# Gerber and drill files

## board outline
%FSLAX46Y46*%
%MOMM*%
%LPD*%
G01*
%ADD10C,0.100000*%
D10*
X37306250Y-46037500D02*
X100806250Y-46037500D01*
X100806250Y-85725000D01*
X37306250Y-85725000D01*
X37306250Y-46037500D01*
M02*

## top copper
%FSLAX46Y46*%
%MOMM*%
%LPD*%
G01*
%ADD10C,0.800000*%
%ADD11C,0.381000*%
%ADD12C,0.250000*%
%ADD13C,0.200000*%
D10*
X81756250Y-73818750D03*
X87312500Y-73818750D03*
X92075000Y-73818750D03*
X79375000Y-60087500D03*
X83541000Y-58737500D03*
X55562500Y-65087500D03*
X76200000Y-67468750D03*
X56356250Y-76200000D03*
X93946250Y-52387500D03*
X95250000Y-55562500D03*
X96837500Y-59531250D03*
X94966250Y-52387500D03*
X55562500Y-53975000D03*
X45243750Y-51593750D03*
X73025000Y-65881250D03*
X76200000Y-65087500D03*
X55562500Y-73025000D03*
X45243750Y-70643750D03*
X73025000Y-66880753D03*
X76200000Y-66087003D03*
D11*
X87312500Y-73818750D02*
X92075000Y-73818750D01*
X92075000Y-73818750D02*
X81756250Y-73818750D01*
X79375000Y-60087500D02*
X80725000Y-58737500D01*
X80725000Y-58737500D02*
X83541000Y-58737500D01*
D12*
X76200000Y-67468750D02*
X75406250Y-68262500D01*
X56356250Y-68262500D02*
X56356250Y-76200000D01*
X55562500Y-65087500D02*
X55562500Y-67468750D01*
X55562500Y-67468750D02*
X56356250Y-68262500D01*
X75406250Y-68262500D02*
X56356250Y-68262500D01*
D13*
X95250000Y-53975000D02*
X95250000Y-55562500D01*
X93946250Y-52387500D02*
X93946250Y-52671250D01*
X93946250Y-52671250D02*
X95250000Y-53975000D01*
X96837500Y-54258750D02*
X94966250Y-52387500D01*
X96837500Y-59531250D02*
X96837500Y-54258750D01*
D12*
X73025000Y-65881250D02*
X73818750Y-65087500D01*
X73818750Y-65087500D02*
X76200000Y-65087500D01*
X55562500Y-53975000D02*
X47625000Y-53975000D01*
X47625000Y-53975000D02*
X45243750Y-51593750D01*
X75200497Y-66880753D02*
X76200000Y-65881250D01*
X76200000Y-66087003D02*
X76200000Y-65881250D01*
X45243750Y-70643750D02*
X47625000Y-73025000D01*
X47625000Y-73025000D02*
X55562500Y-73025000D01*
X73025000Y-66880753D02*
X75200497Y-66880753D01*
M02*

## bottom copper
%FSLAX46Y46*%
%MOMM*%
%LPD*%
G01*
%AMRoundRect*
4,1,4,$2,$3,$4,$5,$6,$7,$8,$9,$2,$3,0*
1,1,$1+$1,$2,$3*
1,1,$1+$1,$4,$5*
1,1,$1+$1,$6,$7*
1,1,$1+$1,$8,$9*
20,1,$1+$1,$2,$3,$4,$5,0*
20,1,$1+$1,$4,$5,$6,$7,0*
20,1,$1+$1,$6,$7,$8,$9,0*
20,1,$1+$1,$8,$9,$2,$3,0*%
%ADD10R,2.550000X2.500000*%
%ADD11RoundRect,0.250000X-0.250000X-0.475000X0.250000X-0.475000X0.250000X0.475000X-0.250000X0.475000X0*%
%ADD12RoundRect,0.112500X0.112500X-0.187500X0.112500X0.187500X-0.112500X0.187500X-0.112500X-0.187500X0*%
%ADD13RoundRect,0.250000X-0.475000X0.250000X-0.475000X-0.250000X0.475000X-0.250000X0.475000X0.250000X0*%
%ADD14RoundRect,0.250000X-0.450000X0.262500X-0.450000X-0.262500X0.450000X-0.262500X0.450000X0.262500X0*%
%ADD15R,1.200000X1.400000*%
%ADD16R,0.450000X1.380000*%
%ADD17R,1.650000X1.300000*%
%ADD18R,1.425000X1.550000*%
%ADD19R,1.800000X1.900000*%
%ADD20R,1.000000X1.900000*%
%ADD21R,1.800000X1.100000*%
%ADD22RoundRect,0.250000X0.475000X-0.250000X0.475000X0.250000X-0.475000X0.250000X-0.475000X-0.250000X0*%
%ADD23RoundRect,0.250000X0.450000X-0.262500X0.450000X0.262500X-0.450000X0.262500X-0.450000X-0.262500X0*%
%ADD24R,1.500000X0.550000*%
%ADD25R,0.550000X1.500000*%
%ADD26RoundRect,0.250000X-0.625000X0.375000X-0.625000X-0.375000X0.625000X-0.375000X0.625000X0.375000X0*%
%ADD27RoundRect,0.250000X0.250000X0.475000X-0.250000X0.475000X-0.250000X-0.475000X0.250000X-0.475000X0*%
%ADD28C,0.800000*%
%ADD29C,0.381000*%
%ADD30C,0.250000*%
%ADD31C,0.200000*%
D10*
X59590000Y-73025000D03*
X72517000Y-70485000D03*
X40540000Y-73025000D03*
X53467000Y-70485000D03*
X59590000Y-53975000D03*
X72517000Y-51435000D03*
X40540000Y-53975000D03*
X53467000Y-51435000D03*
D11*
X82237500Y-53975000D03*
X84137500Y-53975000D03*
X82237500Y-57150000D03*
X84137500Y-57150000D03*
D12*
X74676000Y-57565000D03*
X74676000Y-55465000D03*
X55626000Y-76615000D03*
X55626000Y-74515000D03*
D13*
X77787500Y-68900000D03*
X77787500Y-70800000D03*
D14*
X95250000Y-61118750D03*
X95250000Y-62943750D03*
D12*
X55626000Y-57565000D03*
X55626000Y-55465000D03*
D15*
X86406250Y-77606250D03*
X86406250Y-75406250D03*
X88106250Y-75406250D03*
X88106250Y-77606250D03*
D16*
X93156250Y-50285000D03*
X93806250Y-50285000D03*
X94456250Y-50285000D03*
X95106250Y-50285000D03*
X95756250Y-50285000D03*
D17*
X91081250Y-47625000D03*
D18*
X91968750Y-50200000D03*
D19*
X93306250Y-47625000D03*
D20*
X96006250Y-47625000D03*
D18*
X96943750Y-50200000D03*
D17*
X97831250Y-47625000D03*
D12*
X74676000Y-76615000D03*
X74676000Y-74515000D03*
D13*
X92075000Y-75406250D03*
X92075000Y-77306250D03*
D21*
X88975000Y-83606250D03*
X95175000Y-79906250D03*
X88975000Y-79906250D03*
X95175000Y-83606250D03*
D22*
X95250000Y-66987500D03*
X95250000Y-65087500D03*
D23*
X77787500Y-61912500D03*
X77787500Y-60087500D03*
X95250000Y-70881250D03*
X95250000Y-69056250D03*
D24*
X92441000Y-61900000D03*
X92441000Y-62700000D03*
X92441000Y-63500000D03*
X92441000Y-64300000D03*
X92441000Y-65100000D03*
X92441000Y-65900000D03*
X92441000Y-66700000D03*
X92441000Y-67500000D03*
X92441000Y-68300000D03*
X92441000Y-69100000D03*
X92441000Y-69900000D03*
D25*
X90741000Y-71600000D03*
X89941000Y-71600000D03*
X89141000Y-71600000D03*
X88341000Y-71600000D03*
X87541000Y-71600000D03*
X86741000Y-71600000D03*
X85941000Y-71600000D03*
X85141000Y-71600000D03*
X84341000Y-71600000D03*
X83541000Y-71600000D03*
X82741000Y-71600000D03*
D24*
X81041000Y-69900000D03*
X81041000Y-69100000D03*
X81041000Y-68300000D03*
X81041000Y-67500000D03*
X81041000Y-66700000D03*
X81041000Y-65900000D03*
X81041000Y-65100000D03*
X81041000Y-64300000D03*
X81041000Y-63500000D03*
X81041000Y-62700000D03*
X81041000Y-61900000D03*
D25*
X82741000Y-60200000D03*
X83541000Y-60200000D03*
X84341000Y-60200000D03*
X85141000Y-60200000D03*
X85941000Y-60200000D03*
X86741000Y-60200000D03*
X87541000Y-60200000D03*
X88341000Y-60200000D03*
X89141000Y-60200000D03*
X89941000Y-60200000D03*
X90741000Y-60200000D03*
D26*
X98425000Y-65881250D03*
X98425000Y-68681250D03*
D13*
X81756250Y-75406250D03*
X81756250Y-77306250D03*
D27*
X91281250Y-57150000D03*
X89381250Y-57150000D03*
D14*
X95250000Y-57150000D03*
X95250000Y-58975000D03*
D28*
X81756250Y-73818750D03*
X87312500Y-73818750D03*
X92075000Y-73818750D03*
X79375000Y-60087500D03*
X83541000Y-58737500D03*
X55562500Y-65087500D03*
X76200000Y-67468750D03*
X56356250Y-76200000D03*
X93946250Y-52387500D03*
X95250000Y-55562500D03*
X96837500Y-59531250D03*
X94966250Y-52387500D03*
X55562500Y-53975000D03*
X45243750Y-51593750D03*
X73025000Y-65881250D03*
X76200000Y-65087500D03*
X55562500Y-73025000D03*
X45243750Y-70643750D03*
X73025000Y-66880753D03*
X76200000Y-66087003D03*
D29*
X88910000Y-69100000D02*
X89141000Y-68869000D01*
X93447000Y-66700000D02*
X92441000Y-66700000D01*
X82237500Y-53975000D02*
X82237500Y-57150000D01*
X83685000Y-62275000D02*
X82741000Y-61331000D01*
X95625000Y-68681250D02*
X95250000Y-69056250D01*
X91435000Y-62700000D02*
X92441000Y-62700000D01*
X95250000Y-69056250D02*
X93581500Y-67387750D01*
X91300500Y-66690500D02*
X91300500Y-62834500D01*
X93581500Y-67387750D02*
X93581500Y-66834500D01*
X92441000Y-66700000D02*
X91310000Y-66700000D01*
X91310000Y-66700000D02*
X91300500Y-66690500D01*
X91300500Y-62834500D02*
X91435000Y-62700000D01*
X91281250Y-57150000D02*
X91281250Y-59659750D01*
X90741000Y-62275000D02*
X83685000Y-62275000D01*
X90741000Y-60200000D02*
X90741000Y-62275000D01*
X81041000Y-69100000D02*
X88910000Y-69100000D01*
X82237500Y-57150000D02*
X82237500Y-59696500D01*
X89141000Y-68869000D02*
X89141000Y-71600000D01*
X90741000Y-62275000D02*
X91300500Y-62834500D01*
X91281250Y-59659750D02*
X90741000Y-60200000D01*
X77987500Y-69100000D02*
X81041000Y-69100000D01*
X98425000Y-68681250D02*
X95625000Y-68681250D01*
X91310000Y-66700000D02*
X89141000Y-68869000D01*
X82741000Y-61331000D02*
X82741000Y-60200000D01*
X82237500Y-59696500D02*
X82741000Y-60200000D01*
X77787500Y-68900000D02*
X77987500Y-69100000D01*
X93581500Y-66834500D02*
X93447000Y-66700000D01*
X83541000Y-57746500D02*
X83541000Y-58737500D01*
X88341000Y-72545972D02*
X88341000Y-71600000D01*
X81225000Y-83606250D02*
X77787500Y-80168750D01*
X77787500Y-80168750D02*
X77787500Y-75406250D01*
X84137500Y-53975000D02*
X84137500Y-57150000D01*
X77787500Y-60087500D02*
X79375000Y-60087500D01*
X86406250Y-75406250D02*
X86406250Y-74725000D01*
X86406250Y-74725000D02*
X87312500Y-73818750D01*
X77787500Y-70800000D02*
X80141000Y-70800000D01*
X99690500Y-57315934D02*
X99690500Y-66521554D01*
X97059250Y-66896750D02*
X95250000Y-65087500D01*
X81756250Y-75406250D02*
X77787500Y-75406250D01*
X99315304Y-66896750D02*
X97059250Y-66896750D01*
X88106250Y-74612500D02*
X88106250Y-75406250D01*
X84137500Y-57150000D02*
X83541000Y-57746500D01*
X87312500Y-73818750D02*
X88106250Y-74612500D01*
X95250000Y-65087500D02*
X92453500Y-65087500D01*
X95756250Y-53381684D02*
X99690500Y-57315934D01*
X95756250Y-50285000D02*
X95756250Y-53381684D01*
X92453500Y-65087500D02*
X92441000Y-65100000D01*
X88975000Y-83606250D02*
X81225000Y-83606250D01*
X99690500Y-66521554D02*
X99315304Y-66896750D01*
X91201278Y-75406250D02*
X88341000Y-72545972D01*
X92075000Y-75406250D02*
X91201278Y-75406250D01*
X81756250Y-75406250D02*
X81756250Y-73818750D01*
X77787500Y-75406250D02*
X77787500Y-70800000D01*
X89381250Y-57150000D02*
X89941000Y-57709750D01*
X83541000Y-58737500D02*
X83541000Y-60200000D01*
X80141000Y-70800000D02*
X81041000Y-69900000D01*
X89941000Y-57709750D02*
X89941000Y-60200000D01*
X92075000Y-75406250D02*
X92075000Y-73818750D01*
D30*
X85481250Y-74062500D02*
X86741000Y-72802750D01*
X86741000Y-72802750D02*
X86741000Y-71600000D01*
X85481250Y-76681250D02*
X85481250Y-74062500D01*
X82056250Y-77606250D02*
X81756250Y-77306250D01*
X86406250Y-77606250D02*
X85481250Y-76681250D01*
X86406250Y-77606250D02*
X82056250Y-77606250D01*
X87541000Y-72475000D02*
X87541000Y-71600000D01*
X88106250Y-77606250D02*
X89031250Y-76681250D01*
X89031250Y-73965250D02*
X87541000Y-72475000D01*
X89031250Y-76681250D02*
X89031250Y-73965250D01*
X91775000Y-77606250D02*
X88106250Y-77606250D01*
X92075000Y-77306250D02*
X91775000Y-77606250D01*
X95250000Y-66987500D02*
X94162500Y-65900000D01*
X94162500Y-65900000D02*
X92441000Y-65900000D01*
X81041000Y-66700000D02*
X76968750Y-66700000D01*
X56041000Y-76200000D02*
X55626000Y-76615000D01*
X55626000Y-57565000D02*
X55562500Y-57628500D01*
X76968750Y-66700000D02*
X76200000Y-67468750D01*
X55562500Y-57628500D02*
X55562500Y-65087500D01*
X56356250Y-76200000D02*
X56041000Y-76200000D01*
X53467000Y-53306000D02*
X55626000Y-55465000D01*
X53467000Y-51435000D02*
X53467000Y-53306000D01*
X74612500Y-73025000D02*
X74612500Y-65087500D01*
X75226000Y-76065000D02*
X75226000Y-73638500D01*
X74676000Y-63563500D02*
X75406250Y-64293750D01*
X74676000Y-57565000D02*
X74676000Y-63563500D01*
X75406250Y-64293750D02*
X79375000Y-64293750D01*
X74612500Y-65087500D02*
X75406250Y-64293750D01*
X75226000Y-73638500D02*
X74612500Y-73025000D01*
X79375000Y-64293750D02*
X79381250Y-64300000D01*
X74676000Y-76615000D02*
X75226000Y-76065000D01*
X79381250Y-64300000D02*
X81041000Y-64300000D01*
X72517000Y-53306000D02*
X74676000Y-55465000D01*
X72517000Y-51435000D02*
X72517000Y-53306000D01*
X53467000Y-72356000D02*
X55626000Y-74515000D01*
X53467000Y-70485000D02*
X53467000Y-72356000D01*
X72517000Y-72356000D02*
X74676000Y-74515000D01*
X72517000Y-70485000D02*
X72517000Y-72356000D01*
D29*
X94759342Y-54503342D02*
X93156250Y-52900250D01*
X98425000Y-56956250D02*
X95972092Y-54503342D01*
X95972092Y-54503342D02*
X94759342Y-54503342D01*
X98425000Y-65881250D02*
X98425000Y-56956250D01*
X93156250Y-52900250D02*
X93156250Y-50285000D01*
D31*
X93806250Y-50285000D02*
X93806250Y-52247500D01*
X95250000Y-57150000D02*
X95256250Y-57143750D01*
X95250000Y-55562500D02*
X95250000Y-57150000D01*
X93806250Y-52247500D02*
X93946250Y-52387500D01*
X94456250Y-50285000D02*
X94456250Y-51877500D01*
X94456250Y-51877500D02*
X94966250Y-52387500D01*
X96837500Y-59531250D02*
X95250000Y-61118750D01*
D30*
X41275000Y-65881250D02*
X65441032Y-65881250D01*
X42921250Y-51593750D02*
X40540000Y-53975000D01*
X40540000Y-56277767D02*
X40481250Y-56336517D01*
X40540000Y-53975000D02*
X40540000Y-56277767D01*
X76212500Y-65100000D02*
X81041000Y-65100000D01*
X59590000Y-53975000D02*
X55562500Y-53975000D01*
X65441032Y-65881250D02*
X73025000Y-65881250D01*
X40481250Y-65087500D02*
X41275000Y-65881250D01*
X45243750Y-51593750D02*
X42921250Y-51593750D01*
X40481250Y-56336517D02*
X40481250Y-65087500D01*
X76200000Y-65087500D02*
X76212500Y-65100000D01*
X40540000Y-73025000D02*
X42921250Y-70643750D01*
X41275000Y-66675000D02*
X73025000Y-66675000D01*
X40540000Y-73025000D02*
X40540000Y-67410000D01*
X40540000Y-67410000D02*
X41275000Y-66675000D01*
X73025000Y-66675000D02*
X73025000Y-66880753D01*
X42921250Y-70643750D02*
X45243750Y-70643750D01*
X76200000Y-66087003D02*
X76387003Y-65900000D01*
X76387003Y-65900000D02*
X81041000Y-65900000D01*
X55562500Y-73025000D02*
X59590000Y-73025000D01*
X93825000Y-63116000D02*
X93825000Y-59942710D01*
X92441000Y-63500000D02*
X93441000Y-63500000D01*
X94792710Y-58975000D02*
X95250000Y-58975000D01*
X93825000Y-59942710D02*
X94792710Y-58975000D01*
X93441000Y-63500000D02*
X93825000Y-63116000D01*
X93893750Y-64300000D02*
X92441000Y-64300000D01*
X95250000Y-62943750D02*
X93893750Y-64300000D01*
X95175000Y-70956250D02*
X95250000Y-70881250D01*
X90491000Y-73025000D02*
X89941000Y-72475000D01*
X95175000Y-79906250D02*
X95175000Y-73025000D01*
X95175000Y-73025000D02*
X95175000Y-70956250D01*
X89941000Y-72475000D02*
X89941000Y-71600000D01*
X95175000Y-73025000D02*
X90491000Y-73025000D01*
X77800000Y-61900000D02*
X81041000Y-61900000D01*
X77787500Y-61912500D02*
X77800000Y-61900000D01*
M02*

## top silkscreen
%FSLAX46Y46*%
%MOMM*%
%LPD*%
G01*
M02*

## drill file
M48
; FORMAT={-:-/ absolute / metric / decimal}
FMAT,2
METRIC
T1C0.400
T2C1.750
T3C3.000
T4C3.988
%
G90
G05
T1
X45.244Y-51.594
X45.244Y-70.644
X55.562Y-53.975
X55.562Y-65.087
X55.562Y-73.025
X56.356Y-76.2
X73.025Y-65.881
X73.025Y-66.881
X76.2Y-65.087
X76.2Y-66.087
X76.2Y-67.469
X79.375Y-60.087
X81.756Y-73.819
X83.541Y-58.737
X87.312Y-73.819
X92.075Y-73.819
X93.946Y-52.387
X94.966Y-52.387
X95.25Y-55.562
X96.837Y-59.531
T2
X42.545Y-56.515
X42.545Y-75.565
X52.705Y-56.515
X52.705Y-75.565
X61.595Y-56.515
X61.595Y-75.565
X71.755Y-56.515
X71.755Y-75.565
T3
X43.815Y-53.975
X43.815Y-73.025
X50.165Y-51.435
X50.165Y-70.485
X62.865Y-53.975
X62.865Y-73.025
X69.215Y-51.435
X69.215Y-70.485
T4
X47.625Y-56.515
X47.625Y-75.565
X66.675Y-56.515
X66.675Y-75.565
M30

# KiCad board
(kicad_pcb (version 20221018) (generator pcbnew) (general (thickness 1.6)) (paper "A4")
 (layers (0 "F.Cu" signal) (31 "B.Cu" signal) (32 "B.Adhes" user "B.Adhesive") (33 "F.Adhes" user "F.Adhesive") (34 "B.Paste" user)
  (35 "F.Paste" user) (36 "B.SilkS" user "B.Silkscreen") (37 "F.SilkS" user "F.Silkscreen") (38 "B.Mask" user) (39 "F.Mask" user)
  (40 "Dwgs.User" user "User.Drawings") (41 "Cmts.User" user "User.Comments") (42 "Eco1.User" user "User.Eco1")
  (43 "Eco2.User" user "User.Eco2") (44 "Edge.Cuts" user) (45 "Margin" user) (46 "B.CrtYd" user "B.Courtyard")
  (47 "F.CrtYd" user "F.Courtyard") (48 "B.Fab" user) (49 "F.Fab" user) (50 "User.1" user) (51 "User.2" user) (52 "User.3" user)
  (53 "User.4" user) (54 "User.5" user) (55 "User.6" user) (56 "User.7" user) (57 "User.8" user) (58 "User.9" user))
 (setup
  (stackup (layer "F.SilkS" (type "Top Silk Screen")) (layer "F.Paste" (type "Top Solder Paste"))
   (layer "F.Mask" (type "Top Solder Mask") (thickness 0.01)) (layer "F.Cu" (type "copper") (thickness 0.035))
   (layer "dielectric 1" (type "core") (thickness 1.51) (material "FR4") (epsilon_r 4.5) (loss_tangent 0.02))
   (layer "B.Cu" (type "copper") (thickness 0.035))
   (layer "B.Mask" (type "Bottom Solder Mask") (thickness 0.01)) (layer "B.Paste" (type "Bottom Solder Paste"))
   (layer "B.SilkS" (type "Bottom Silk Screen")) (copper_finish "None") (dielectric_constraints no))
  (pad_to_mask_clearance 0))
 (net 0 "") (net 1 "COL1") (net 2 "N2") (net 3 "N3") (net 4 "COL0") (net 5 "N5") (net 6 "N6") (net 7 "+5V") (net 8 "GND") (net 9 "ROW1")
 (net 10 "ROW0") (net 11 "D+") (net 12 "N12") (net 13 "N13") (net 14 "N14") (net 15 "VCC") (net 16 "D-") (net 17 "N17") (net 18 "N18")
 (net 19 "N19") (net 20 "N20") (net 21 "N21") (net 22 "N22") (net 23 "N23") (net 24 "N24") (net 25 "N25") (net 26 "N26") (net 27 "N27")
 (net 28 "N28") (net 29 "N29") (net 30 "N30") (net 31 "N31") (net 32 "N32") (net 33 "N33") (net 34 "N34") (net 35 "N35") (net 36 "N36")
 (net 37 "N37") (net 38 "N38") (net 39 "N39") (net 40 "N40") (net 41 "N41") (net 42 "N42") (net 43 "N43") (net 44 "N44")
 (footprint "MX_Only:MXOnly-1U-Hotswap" (layer "F.Cu") (at 66.675 75.565)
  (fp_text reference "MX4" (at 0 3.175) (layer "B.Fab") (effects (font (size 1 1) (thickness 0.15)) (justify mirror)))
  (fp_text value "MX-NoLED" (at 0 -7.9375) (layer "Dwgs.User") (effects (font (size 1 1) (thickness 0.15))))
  (pad "" np_thru_hole circle (at -5.08 0 48.0996) (size 1.75 1.75) (drill 1.75) (layers "*.Cu" "*.Mask"))
  (pad "" np_thru_hole circle (at -3.81 -2.54) (size 3 3) (drill 3) (layers "*.Cu" "*.Mask"))
  (pad "" np_thru_hole circle (at 0 0) (size 3.9878 3.9878) (drill 3.9878) (layers "*.Cu" "*.Mask"))
  (pad "" np_thru_hole circle (at 2.54 -5.08) (size 3 3) (drill 3) (layers "*.Cu" "*.Mask"))
  (pad "" np_thru_hole circle (at 5.08 0 48.0996) (size 1.75 1.75) (drill 1.75) (layers "*.Cu" "*.Mask"))
  (pad "1" smd rect (at -7.085 -2.54) (size 2.55 2.5) (layers "B.Cu" "B.Paste" "B.Mask") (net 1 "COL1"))
  (pad "2" smd rect (at 5.842 -5.08) (size 2.55 2.5) (layers "B.Cu" "B.Paste" "B.Mask") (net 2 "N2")))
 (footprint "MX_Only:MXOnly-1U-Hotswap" (layer "F.Cu") (at 47.625 75.565)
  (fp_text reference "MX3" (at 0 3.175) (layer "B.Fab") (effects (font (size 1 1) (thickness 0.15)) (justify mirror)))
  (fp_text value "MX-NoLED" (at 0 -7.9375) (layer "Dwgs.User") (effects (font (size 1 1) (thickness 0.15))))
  (pad "" np_thru_hole circle (at -5.08 0 48.0996) (size 1.75 1.75) (drill 1.75) (layers "*.Cu" "*.Mask"))
  (pad "" np_thru_hole circle (at -3.81 -2.54) (size 3 3) (drill 3) (layers "*.Cu" "*.Mask"))
  (pad "" np_thru_hole circle (at 0 0) (size 3.9878 3.9878) (drill 3.9878) (layers "*.Cu" "*.Mask"))
  (pad "" np_thru_hole circle (at 2.54 -5.08) (size 3 3) (drill 3) (layers "*.Cu" "*.Mask"))
  (pad "" np_thru_hole circle (at 5.08 0 48.0996) (size 1.75 1.75) (drill 1.75) (layers "*.Cu" "*.Mask"))
  (pad "1" smd rect (at -7.085 -2.54) (size 2.55 2.5) (layers "B.Cu" "B.Paste" "B.Mask") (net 1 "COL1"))
  (pad "2" smd rect (at 5.842 -5.08) (size 2.55 2.5) (layers "B.Cu" "B.Paste" "B.Mask") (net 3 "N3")))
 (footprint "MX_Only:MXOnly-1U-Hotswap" (layer "F.Cu") (at 66.675 56.515)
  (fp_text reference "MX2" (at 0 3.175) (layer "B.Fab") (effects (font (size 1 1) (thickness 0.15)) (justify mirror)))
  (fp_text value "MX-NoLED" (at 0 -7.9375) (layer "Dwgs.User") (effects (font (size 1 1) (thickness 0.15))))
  (pad "" np_thru_hole circle (at -5.08 0 48.0996) (size 1.75 1.75) (drill 1.75) (layers "*.Cu" "*.Mask"))
  (pad "" np_thru_hole circle (at -3.81 -2.54) (size 3 3) (drill 3) (layers "*.Cu" "*.Mask"))
  (pad "" np_thru_hole circle (at 0 0) (size 3.9878 3.9878) (drill 3.9878) (layers "*.Cu" "*.Mask"))
  (pad "" np_thru_hole circle (at 2.54 -5.08) (size 3 3) (drill 3) (layers "*.Cu" "*.Mask"))
  (pad "" np_thru_hole circle (at 5.08 0 48.0996) (size 1.75 1.75) (drill 1.75) (layers "*.Cu" "*.Mask"))
  (pad "1" smd rect (at -7.085 -2.54) (size 2.55 2.5) (layers "B.Cu" "B.Paste" "B.Mask") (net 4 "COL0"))
  (pad "2" smd rect (at 5.842 -5.08) (size 2.55 2.5) (layers "B.Cu" "B.Paste" "B.Mask") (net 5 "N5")))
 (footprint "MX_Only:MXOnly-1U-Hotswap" (layer "F.Cu") (at 47.625 56.515)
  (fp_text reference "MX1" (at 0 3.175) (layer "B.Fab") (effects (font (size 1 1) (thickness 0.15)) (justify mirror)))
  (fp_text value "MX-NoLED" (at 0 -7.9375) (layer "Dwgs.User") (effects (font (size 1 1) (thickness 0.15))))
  (pad "" np_thru_hole circle (at -5.08 0 48.0996) (size 1.75 1.75) (drill 1.75) (layers "*.Cu" "*.Mask"))
  (pad "" np_thru_hole circle (at -3.81 -2.54) (size 3 3) (drill 3) (layers "*.Cu" "*.Mask"))
  (pad "" np_thru_hole circle (at 0 0) (size 3.9878 3.9878) (drill 3.9878) (layers "*.Cu" "*.Mask"))
  (pad "" np_thru_hole circle (at 2.54 -5.08) (size 3 3) (drill 3) (layers "*.Cu" "*.Mask"))
  (pad "" np_thru_hole circle (at 5.08 0 48.0996) (size 1.75 1.75) (drill 1.75) (layers "*.Cu" "*.Mask"))
  (pad "1" smd rect (at -7.085 -2.54) (size 2.55 2.5) (layers "B.Cu" "B.Paste" "B.Mask") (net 4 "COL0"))
  (pad "2" smd rect (at 5.842 -5.08) (size 2.55 2.5) (layers "B.Cu" "B.Paste" "B.Mask") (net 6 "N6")))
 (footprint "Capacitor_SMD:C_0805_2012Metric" (layer "B.Cu") (at 83.1875 53.975)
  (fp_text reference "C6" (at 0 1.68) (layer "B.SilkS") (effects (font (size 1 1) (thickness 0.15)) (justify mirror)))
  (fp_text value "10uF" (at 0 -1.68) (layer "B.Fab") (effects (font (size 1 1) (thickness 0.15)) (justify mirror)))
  (pad "1" smd roundrect (at -0.95 0) (size 1 1.45) (layers "B.Cu" "B.Paste" "B.Mask") (roundrect_rratio 0.25) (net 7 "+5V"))
  (pad "2" smd roundrect (at 0.95 0) (size 1 1.45) (layers "B.Cu" "B.Paste" "B.Mask") (roundrect_rratio 0.25) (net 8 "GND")))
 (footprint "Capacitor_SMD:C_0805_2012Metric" (layer "B.Cu") (at 83.1875 57.15)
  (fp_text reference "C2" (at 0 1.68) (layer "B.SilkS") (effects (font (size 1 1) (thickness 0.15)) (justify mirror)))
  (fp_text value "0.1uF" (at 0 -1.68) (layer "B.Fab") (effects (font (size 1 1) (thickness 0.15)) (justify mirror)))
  (pad "1" smd roundrect (at -0.95 0) (size 1 1.45) (layers "B.Cu" "B.Paste" "B.Mask") (roundrect_rratio 0.25) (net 7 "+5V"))
  (pad "2" smd roundrect (at 0.95 0) (size 1 1.45) (layers "B.Cu" "B.Paste" "B.Mask") (roundrect_rratio 0.25) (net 8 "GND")))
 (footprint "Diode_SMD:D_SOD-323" (layer "B.Cu") (at 74.676 56.515 90)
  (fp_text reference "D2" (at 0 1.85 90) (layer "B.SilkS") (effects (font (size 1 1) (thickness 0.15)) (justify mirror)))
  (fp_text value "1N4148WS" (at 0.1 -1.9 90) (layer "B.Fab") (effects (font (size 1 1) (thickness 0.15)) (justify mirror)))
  (pad "1" smd roundrect (at -1.05 0 90) (size 0.6 0.45) (layers "B.Cu" "B.Paste" "B.Mask") (roundrect_rratio 0.25) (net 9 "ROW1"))
  (pad "2" smd roundrect (at 1.05 0 90) (size 0.6 0.45) (layers "B.Cu" "B.Paste" "B.Mask") (roundrect_rratio 0.25) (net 5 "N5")))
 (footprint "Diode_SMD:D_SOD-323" (layer "B.Cu") (at 55.626 75.565 90)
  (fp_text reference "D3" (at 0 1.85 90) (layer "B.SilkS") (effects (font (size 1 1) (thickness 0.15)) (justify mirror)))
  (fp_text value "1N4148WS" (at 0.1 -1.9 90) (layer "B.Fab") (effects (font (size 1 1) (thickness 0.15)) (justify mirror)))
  (pad "1" smd roundrect (at -1.05 0 90) (size 0.6 0.45) (layers "B.Cu" "B.Paste" "B.Mask") (roundrect_rratio 0.25) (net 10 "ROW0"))
  (pad "2" smd roundrect (at 1.05 0 90) (size 0.6 0.45) (layers "B.Cu" "B.Paste" "B.Mask") (roundrect_rratio 0.25) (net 3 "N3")))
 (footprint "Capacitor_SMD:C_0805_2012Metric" (layer "B.Cu") (at 77.7875 69.85 -90)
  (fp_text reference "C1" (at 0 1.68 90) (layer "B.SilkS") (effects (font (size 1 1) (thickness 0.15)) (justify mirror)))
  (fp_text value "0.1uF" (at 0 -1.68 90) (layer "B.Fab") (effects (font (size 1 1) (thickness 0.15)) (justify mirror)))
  (pad "1" smd roundrect (at -0.95 0 270) (size 1 1.45) (layers "B.Cu" "B.Paste" "B.Mask") (roundrect_rratio 0.25) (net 7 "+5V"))
  (pad "2" smd roundrect (at 0.95 0 270) (size 1 1.45) (layers "B.Cu" "B.Paste" "B.Mask") (roundrect_rratio 0.25) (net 8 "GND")))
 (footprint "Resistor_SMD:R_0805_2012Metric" (layer "B.Cu") (at 95.25 62.03125 -90)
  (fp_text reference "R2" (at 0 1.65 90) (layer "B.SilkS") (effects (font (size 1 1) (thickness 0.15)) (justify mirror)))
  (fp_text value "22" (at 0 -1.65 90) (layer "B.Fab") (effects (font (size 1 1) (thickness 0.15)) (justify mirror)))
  (pad "1" smd roundrect (at -0.9125 0 270) (size 1.025 1.4) (layers "B.Cu" "B.Paste" "B.Mask") (roundrect_rratio 0.243902) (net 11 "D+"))
  (pad "2" smd roundrect (at 0.9125 0 270) (size 1.025 1.4) (layers "B.Cu" "B.Paste" "B.Mask") (roundrect_rratio 0.243902) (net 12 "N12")))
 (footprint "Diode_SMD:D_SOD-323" (layer "B.Cu") (at 55.626 56.515 90)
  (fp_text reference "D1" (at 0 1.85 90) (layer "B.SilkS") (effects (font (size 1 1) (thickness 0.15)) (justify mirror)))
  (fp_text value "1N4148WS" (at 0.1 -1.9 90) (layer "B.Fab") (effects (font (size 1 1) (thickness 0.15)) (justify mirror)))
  (pad "1" smd roundrect (at -1.05 0 90) (size 0.6 0.45) (layers "B.Cu" "B.Paste" "B.Mask") (roundrect_rratio 0.25) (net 10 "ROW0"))
  (pad "2" smd roundrect (at 1.05 0 90) (size 0.6 0.45) (layers "B.Cu" "B.Paste" "B.Mask") (roundrect_rratio 0.25) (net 6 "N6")))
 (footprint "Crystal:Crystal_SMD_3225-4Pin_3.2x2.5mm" (layer "B.Cu") (at 87.25625 76.50625 90)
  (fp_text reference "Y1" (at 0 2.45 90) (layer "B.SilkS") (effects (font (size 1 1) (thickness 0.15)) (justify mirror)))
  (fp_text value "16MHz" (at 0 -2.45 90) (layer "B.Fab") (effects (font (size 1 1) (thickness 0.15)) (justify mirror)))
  (pad "1" smd rect (at -1.1 -0.85 90) (size 1.4 1.2) (layers "B.Cu" "B.Paste" "B.Mask") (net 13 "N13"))
  (pad "2" smd rect (at 1.1 -0.85 90) (size 1.4 1.2) (layers "B.Cu" "B.Paste" "B.Mask") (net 8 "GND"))
  (pad "3" smd rect (at 1.1 0.85 90) (size 1.4 1.2) (layers "B.Cu" "B.Paste" "B.Mask") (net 8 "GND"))
  (pad "4" smd rect (at -1.1 0.85 90) (size 1.4 1.2) (layers "B.Cu" "B.Paste" "B.Mask") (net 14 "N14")))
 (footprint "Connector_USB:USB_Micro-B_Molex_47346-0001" (layer "B.Cu") (at 94.45625 48.825)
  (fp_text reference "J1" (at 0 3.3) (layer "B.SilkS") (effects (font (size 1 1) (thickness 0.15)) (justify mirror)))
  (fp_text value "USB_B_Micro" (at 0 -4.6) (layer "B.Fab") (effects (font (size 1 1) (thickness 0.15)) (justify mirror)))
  (pad "1" smd rect (at -1.3 1.46) (size 0.45 1.38) (layers "B.Cu" "B.Paste" "B.Mask") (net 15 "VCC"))
  (pad "2" smd rect (at -0.65 1.46) (size 0.45 1.38) (layers "B.Cu" "B.Paste" "B.Mask") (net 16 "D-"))
  (pad "3" smd rect (at 0 1.46) (size 0.45 1.38) (layers "B.Cu" "B.Paste" "B.Mask") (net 11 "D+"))
  (pad "4" smd rect (at 0.65 1.46) (size 0.45 1.38) (layers "B.Cu" "B.Paste" "B.Mask") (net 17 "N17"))
  (pad "5" smd rect (at 1.3 1.46) (size 0.45 1.38) (layers "B.Cu" "B.Paste" "B.Mask") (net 8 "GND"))
  (pad "6" smd rect (at -3.375 -1.2) (size 1.65 1.3) (layers "B.Cu" "B.Paste" "B.Mask") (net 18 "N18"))
  (pad "6" smd rect (at -2.4875 1.375) (size 1.425 1.55) (layers "B.Cu" "B.Paste" "B.Mask") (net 18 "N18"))
  (pad "6" smd rect (at -1.15 -1.2) (size 1.8 1.9) (layers "B.Cu" "B.Paste" "B.Mask") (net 18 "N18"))
  (pad "6" smd rect (at 1.55 -1.2) (size 1 1.9) (layers "B.Cu" "B.Paste" "B.Mask") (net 18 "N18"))
  (pad "6" smd rect (at 2.4875 1.375) (size 1.425 1.55) (layers "B.Cu" "B.Paste" "B.Mask") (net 18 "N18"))
  (pad "6" smd rect (at 3.375 -1.2) (size 1.65 1.3) (layers "B.Cu" "B.Paste" "B.Mask") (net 18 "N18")))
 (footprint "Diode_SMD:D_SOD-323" (layer "B.Cu") (at 74.676 75.565 90)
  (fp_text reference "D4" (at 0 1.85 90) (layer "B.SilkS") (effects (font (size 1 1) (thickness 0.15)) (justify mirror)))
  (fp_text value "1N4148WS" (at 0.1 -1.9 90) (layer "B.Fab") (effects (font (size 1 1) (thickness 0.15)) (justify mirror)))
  (pad "1" smd roundrect (at -1.05 0 90) (size 0.6 0.45) (layers "B.Cu" "B.Paste" "B.Mask") (roundrect_rratio 0.25) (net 9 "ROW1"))
  (pad "2" smd roundrect (at 1.05 0 90) (size 0.6 0.45) (layers "B.Cu" "B.Paste" "B.Mask") (roundrect_rratio 0.25) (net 2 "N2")))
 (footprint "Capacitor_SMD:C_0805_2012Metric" (layer "B.Cu") (at 92.075 76.35625 -90)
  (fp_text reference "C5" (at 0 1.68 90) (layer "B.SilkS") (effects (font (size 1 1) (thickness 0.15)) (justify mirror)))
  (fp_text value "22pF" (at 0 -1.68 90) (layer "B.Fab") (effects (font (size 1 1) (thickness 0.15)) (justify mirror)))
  (pad "1" smd roundrect (at -0.95 0 270) (size 1 1.45) (layers "B.Cu" "B.Paste" "B.Mask") (roundrect_rratio 0.25) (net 8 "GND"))
  (pad "2" smd roundrect (at 0.95 0 270) (size 1 1.45) (layers "B.Cu" "B.Paste" "B.Mask") (roundrect_rratio 0.25) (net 14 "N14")))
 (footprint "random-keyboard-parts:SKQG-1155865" (layer "B.Cu") (at 92.075 81.75625 180)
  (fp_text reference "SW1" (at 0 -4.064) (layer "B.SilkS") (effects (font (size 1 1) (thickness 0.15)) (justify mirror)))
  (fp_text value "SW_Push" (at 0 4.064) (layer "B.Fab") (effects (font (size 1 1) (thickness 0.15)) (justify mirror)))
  (pad "1" smd rect (at 3.1 -1.85 180) (size 1.8 1.1) (layers "B.Cu" "B.Paste" "B.Mask") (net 8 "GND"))
  (pad "2" smd rect (at -3.1 1.85 180) (size 1.8 1.1) (layers "B.Cu" "B.Paste" "B.Mask") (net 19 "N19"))
  (pad "3" smd rect (at 3.1 1.85 180) (size 1.8 1.1) (layers "B.Cu" "B.Paste" "B.Mask"))
  (pad "4" smd rect (at -3.1 -1.85 180) (size 1.8 1.1) (layers "B.Cu" "B.Paste" "B.Mask")))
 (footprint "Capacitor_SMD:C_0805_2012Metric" (layer "B.Cu") (at 95.25 66.0375 90)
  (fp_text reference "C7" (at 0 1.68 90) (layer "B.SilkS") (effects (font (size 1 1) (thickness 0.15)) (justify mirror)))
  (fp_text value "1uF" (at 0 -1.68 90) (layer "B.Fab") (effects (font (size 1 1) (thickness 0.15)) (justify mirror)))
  (pad "1" smd roundrect (at -0.95 0 90) (size 1 1.45) (layers "B.Cu" "B.Paste" "B.Mask") (roundrect_rratio 0.25) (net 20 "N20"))
  (pad "2" smd roundrect (at 0.95 0 90) (size 1 1.45) (layers "B.Cu" "B.Paste" "B.Mask") (roundrect_rratio 0.25) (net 8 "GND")))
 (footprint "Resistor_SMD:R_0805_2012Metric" (layer "B.Cu") (at 77.7875 61 90)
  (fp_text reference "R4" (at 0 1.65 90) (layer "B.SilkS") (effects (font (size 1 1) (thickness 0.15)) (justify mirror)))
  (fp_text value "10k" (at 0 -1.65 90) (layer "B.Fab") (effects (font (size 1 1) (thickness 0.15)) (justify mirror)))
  (pad "1" smd roundrect (at -0.9125 0 90) (size 1.025 1.4) (layers "B.Cu" "B.Paste" "B.Mask") (roundrect_rratio 0.243902) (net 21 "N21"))
  (pad "2" smd roundrect (at 0.9125 0 90) (size 1.025 1.4) (layers "B.Cu" "B.Paste" "B.Mask") (roundrect_rratio 0.243902) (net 8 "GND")))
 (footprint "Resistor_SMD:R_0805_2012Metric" (layer "B.Cu") (at 95.25 69.96875 90)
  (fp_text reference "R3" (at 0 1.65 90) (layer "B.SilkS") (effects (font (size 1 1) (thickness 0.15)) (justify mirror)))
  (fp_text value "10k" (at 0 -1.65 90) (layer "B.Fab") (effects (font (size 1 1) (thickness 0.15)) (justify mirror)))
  (pad "1" smd roundrect (at -0.9125 0 90) (size 1.025 1.4) (layers "B.Cu" "B.Paste" "B.Mask") (roundrect_rratio 0.243902) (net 19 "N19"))
  (pad "2" smd roundrect (at 0.9125 0 90) (size 1.025 1.4) (layers "B.Cu" "B.Paste" "B.Mask") (roundrect_rratio 0.243902) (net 7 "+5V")))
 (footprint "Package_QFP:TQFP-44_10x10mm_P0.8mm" (layer "B.Cu") (at 86.741 65.9 180)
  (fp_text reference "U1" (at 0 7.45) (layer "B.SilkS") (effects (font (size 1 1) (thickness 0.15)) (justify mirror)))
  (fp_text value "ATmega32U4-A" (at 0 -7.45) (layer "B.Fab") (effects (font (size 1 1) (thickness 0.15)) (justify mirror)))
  (pad "1" smd rect (at -5.7 4 180) (size 1.5 0.55) (layers "B.Cu" "B.Paste" "B.Mask") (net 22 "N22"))
  (pad "2" smd rect (at -5.7 3.2 180) (size 1.5 0.55) (layers "B.Cu" "B.Paste" "B.Mask") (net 7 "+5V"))
  (pad "3" smd rect (at -5.7 2.4 180) (size 1.5 0.55) (layers "B.Cu" "B.Paste" "B.Mask") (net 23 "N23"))
  (pad "4" smd rect (at -5.7 1.6 180) (size 1.5 0.55) (layers "B.Cu" "B.Paste" "B.Mask") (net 12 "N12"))
  (pad "5" smd rect (at -5.7 0.8 180) (size 1.5 0.55) (layers "B.Cu" "B.Paste" "B.Mask") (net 8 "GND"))
  (pad "6" smd rect (at -5.7 0 180) (size 1.5 0.55) (layers "B.Cu" "B.Paste" "B.Mask") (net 20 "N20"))
  (pad "7" smd rect (at -5.7 -0.8 180) (size 1.5 0.55) (layers "B.Cu" "B.Paste" "B.Mask") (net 7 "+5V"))
  (pad "8" smd rect (at -5.7 -1.6 180) (size 1.5 0.55) (layers "B.Cu" "B.Paste" "B.Mask") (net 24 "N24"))
  (pad "9" smd rect (at -5.7 -2.4 180) (size 1.5 0.55) (layers "B.Cu" "B.Paste" "B.Mask") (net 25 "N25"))
  (pad "10" smd rect (at -5.7 -3.2 180) (size 1.5 0.55) (layers "B.Cu" "B.Paste" "B.Mask") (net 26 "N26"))
  (pad "11" smd rect (at -5.7 -4 180) (size 1.5 0.55) (layers "B.Cu" "B.Paste" "B.Mask") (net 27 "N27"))
  (pad "12" smd rect (at -4 -5.7 90) (size 1.5 0.55) (layers "B.Cu" "B.Paste" "B.Mask") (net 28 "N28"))
  (pad "13" smd rect (at -3.2 -5.7 90) (size 1.5 0.55) (layers "B.Cu" "B.Paste" "B.Mask") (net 19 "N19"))
  (pad "14" smd rect (at -2.4 -5.7 90) (size 1.5 0.55) (layers "B.Cu" "B.Paste" "B.Mask") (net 7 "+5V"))
  (pad "15" smd rect (at -1.6 -5.7 90) (size 1.5 0.55) (layers "B.Cu" "B.Paste" "B.Mask") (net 8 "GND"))
  (pad "16" smd rect (at -0.8 -5.7 90) (size 1.5 0.55) (layers "B.Cu" "B.Paste" "B.Mask") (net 14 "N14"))
  (pad "17" smd rect (at 0 -5.7 90) (size 1.5 0.55) (layers "B.Cu" "B.Paste" "B.Mask") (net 13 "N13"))
  (pad "18" smd rect (at 0.8 -5.7 90) (size 1.5 0.55) (layers "B.Cu" "B.Paste" "B.Mask") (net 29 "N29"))
  (pad "19" smd rect (at 1.6 -5.7 90) (size 1.5 0.55) (layers "B.Cu" "B.Paste" "B.Mask") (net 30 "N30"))
  (pad "20" smd rect (at 2.4 -5.7 90) (size 1.5 0.55) (layers "B.Cu" "B.Paste" "B.Mask") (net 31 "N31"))
  (pad "21" smd rect (at 3.2 -5.7 90) (size 1.5 0.55) (layers "B.Cu" "B.Paste" "B.Mask") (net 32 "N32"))
  (pad "22" smd rect (at 4 -5.7 90) (size 1.5 0.55) (layers "B.Cu" "B.Paste" "B.Mask") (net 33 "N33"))
  (pad "23" smd rect (at 5.7 -4 180) (size 1.5 0.55) (layers "B.Cu" "B.Paste" "B.Mask") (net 8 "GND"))
  (pad "24" smd rect (at 5.7 -3.2 180) (size 1.5 0.55) (layers "B.Cu" "B.Paste" "B.Mask") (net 7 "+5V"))
  (pad "25" smd rect (at 5.7 -2.4 180) (size 1.5 0.55) (layers "B.Cu" "B.Paste" "B.Mask") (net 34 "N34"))
  (pad "26" smd rect (at 5.7 -1.6 180) (size 1.5 0.55) (layers "B.Cu" "B.Paste" "B.Mask") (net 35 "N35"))
  (pad "27" smd rect (at 5.7 -0.8 180) (size 1.5 0.55) (layers "B.Cu" "B.Paste" "B.Mask") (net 10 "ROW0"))
  (pad "28" smd rect (at 5.7 0 180) (size 1.5 0.55) (layers "B.Cu" "B.Paste" "B.Mask") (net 1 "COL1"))
  (pad "29" smd rect (at 5.7 0.8 180) (size 1.5 0.55) (layers "B.Cu" "B.Paste" "B.Mask") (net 4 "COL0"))
  (pad "30" smd rect (at 5.7 1.6 180) (size 1.5 0.55) (layers "B.Cu" "B.Paste" "B.Mask") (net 9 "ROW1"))
  (pad "31" smd rect (at 5.7 2.4 180) (size 1.5 0.55) (layers "B.Cu" "B.Paste" "B.Mask") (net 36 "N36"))
  (pad "32" smd rect (at 5.7 3.2 180) (size 1.5 0.55) (layers "B.Cu" "B.Paste" "B.Mask") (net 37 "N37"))
  (pad "33" smd rect (at 5.7 4 180) (size 1.5 0.55) (layers "B.Cu" "B.Paste" "B.Mask") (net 21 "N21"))
  (pad "34" smd rect (at 4 5.7 90) (size 1.5 0.55) (layers "B.Cu" "B.Paste" "B.Mask") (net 7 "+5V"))
  (pad "35" smd rect (at 3.2 5.7 90) (size 1.5 0.55) (layers "B.Cu" "B.Paste" "B.Mask") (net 8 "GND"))
  (pad "36" smd rect (at 2.4 5.7 90) (size 1.5 0.55) (layers "B.Cu" "B.Paste" "B.Mask") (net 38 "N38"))
  (pad "37" smd rect (at 1.6 5.7 90) (size 1.5 0.55) (layers "B.Cu" "B.Paste" "B.Mask") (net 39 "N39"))
  (pad "38" smd rect (at 0.8 5.7 90) (size 1.5 0.55) (layers "B.Cu" "B.Paste" "B.Mask") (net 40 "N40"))
  (pad "39" smd rect (at 0 5.7 90) (size 1.5 0.55) (layers "B.Cu" "B.Paste" "B.Mask") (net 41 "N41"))
  (pad "40" smd rect (at -0.8 5.7 90) (size 1.5 0.55) (layers "B.Cu" "B.Paste" "B.Mask") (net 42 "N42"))
  (pad "41" smd rect (at -1.6 5.7 90) (size 1.5 0.55) (layers "B.Cu" "B.Paste" "B.Mask") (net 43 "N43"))
  (pad "42" smd rect (at -2.4 5.7 90) (size 1.5 0.55) (layers "B.Cu" "B.Paste" "B.Mask") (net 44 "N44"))
  (pad "43" smd rect (at -3.2 5.7 90) (size 1.5 0.55) (layers "B.Cu" "B.Paste" "B.Mask") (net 8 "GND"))
  (pad "44" smd rect (at -4 5.7 90) (size 1.5 0.55) (layers "B.Cu" "B.Paste" "B.Mask") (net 7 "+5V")))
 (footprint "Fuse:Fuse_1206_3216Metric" (layer "B.Cu") (at 98.425 67.28125 -90)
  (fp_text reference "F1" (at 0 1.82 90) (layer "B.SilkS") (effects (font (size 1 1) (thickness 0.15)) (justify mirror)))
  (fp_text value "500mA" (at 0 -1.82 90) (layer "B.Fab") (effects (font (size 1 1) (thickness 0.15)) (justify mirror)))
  (pad "1" smd roundrect (at -1.4 0 270) (size 1.25 1.75) (layers "B.Cu" "B.Paste" "B.Mask") (roundrect_rratio 0.2) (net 15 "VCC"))
  (pad "2" smd roundrect (at 1.4 0 270) (size 1.25 1.75) (layers "B.Cu" "B.Paste" "B.Mask") (roundrect_rratio 0.2) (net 7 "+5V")))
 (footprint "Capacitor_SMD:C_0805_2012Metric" (layer "B.Cu") (at 81.75625 76.35625 -90)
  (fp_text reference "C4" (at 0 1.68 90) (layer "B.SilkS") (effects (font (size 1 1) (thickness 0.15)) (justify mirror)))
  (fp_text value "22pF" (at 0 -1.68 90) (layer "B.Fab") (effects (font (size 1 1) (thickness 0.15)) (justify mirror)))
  (pad "1" smd roundrect (at -0.95 0 270) (size 1 1.45) (layers "B.Cu" "B.Paste" "B.Mask") (roundrect_rratio 0.25) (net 8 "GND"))
  (pad "2" smd roundrect (at 0.95 0 270) (size 1 1.45) (layers "B.Cu" "B.Paste" "B.Mask") (roundrect_rratio 0.25) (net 13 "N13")))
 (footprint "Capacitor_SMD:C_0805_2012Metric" (layer "B.Cu") (at 90.33125 57.15 180)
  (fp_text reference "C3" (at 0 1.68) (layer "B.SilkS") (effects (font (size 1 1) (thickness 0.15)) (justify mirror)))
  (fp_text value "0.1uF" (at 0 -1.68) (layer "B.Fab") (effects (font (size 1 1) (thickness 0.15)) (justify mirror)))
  (pad "1" smd roundrect (at -0.95 0 180) (size 1 1.45) (layers "B.Cu" "B.Paste" "B.Mask") (roundrect_rratio 0.25) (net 7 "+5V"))
  (pad "2" smd roundrect (at 0.95 0 180) (size 1 1.45) (layers "B.Cu" "B.Paste" "B.Mask") (roundrect_rratio 0.25) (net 8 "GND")))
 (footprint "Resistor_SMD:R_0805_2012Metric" (layer "B.Cu") (at 95.25 58.0625 -90)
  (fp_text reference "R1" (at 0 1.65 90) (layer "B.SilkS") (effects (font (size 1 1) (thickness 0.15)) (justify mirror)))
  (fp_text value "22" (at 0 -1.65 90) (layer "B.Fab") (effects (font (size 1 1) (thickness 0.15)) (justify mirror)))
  (pad "1" smd roundrect (at -0.9125 0 270) (size 1.025 1.4) (layers "B.Cu" "B.Paste" "B.Mask") (roundrect_rratio 0.243902) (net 16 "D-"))
  (pad "2" smd roundrect (at 0.9125 0 270) (size 1.025 1.4) (layers "B.Cu" "B.Paste" "B.Mask") (roundrect_rratio 0.243902) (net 23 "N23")))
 (gr_rect (start 37.30625 46.0375) (end 100.80625 85.725) (stroke (width 0.1) (type default)) (fill none) (layer "Edge.Cuts"))
 (segment (start 88.91 69.1) (end 89.141 68.869) (width 0.381) (layer "B.Cu") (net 7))
 (segment (start 93.447 66.7) (end 92.441 66.7) (width 0.381) (layer "B.Cu") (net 7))
 (segment (start 82.2375 53.975) (end 82.2375 57.15) (width 0.381) (layer "B.Cu") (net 7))
 (segment (start 83.685 62.275) (end 82.741 61.331) (width 0.381) (layer "B.Cu") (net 7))
 (segment (start 95.625 68.68125) (end 95.25 69.05625) (width 0.381) (layer "B.Cu") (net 7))
 (segment (start 91.435 62.7) (end 92.441 62.7) (width 0.381) (layer "B.Cu") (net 7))
 (segment (start 95.25 69.05625) (end 93.5815 67.38775) (width 0.381) (layer "B.Cu") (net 7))
 (segment (start 91.3005 66.6905) (end 91.3005 62.8345) (width 0.381) (layer "B.Cu") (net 7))
 (segment (start 93.5815 67.38775) (end 93.5815 66.8345) (width 0.381) (layer "B.Cu") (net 7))
 (segment (start 92.441 66.7) (end 91.31 66.7) (width 0.381) (layer "B.Cu") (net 7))
 (segment (start 91.31 66.7) (end 91.3005 66.6905) (width 0.381) (layer "B.Cu") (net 7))
 (segment (start 91.3005 62.8345) (end 91.435 62.7) (width 0.381) (layer "B.Cu") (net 7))
 (segment (start 91.28125 57.15) (end 91.28125 59.65975) (width 0.381) (layer "B.Cu") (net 7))
 (segment (start 90.741 62.275) (end 83.685 62.275) (width 0.381) (layer "B.Cu") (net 7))
 (segment (start 90.741 60.2) (end 90.741 62.275) (width 0.381) (layer "B.Cu") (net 7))
 (segment (start 81.041 69.1) (end 88.91 69.1) (width 0.381) (layer "B.Cu") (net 7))
 (segment (start 82.2375 57.15) (end 82.2375 59.6965) (width 0.381) (layer "B.Cu") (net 7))
 (segment (start 89.141 68.869) (end 89.141 71.6) (width 0.381) (layer "B.Cu") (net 7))
 (segment (start 90.741 62.275) (end 91.3005 62.8345) (width 0.381) (layer "B.Cu") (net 7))
 (segment (start 91.28125 59.65975) (end 90.741 60.2) (width 0.381) (layer "B.Cu") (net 7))
 (segment (start 77.9875 69.1) (end 81.041 69.1) (width 0.381) (layer "B.Cu") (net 7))
 (segment (start 98.425 68.68125) (end 95.625 68.68125) (width 0.381) (layer "B.Cu") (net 7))
 (segment (start 91.31 66.7) (end 89.141 68.869) (width 0.381) (layer "B.Cu") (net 7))
 (segment (start 82.741 61.331) (end 82.741 60.2) (width 0.381) (layer "B.Cu") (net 7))
 (segment (start 82.2375 59.6965) (end 82.741 60.2) (width 0.381) (layer "B.Cu") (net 7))
 (segment (start 77.7875 68.9) (end 77.9875 69.1) (width 0.381) (layer "B.Cu") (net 7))
 (segment (start 93.5815 66.8345) (end 93.447 66.7) (width 0.381) (layer "B.Cu") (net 7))
 (segment (start 87.3125 73.81875) (end 92.075 73.81875) (width 0.381) (layer "F.Cu") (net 8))
 (segment (start 92.075 73.81875) (end 81.75625 73.81875) (width 0.381) (layer "F.Cu") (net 8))
 (segment (start 79.375 60.0875) (end 80.725 58.7375) (width 0.381) (layer "F.Cu") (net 8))
 (segment (start 80.725 58.7375) (end 83.541 58.7375) (width 0.381) (layer "F.Cu") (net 8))
 (via (at 81.75625 73.81875) (size 0.8) (drill 0.4) (layers "F.Cu" "B.Cu") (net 8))
 (via (at 87.3125 73.81875) (size 0.8) (drill 0.4) (layers "F.Cu" "B.Cu") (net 8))
 (via (at 92.075 73.81875) (size 0.8) (drill 0.4) (layers "F.Cu" "B.Cu") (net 8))
 (via (at 79.375 60.0875) (size 0.8) (drill 0.4) (layers "F.Cu" "B.Cu") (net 8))
 (via (at 83.541 58.7375) (size 0.8) (drill 0.4) (layers "F.Cu" "B.Cu") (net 8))
 (segment (start 83.541 57.7465) (end 83.541 58.7375) (width 0.381) (layer "B.Cu") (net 8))
 (segment (start 88.341 72.545972) (end 88.341 71.6) (width 0.381) (layer "B.Cu") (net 8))
 (segment (start 81.225 83.60625) (end 77.7875 80.16875) (width 0.381) (layer "B.Cu") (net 8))
 (segment (start 77.7875 80.16875) (end 77.7875 75.40625) (width 0.381) (layer "B.Cu") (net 8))
 (segment (start 84.1375 53.975) (end 84.1375 57.15) (width 0.381) (layer "B.Cu") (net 8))
 (segment (start 77.7875 60.0875) (end 79.375 60.0875) (width 0.381) (layer "B.Cu") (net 8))
 (segment (start 86.40625 75.40625) (end 86.40625 74.725) (width 0.381) (layer "B.Cu") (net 8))
 (segment (start 86.40625 74.725) (end 87.3125 73.81875) (width 0.381) (layer "B.Cu") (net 8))
 (segment (start 77.7875 70.8) (end 80.141 70.8) (width 0.381) (layer "B.Cu") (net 8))
 (segment (start 99.6905 57.315934) (end 99.6905 66.521554) (width 0.381) (layer "B.Cu") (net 8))
 (segment (start 97.05925 66.89675) (end 95.25 65.0875) (width 0.381) (layer "B.Cu") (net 8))
 (segment (start 81.75625 75.40625) (end 77.7875 75.40625) (width 0.381) (layer "B.Cu") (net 8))
 (segment (start 99.315304 66.89675) (end 97.05925 66.89675) (width 0.381) (layer "B.Cu") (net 8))
 (segment (start 88.10625 74.6125) (end 88.10625 75.40625) (width 0.381) (layer "B.Cu") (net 8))
 (segment (start 84.1375 57.15) (end 83.541 57.7465) (width 0.381) (layer "B.Cu") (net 8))
 (segment (start 87.3125 73.81875) (end 88.10625 74.6125) (width 0.381) (layer "B.Cu") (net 8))
 (segment (start 95.25 65.0875) (end 92.4535 65.0875) (width 0.381) (layer "B.Cu") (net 8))
 (segment (start 95.75625 53.381684) (end 99.6905 57.315934) (width 0.381) (layer "B.Cu") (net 8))
 (segment (start 95.75625 50.285) (end 95.75625 53.381684) (width 0.381) (layer "B.Cu") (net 8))
 (segment (start 92.4535 65.0875) (end 92.441 65.1) (width 0.381) (layer "B.Cu") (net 8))
 (segment (start 88.975 83.60625) (end 81.225 83.60625) (width 0.381) (layer "B.Cu") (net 8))
 (segment (start 99.6905 66.521554) (end 99.315304 66.89675) (width 0.381) (layer "B.Cu") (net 8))
 (segment (start 91.201278 75.40625) (end 88.341 72.545972) (width 0.381) (layer "B.Cu") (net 8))
 (segment (start 92.075 75.40625) (end 91.201278 75.40625) (width 0.381) (layer "B.Cu") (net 8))
 (segment (start 81.75625 75.40625) (end 81.75625 73.81875) (width 0.381) (layer "B.Cu") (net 8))
 (segment (start 77.7875 75.40625) (end 77.7875 70.8) (width 0.381) (layer "B.Cu") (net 8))
 (segment (start 89.38125 57.15) (end 89.941 57.70975) (width 0.381) (layer "B.Cu") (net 8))
 (segment (start 83.541 58.7375) (end 83.541 60.2) (width 0.381) (layer "B.Cu") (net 8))
 (segment (start 80.141 70.8) (end 81.041 69.9) (width 0.381) (layer "B.Cu") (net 8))
 (segment (start 89.941 57.70975) (end 89.941 60.2) (width 0.381) (layer "B.Cu") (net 8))
 (segment (start 92.075 75.40625) (end 92.075 73.81875) (width 0.381) (layer "B.Cu") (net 8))
 (segment (start 85.48125 74.0625) (end 86.741 72.80275) (width 0.25) (layer "B.Cu") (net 13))
 (segment (start 86.741 72.80275) (end 86.741 71.6) (width 0.25) (layer "B.Cu") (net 13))
 (segment (start 85.48125 76.68125) (end 85.48125 74.0625) (width 0.25) (layer "B.Cu") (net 13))
 (segment (start 82.05625 77.60625) (end 81.75625 77.30625) (width 0.25) (layer "B.Cu") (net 13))
 (segment (start 86.40625 77.60625) (end 85.48125 76.68125) (width 0.25) (layer "B.Cu") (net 13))
 (segment (start 86.40625 77.60625) (end 82.05625 77.60625) (width 0.25) (layer "B.Cu") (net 13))
 (segment (start 87.541 72.475) (end 87.541 71.6) (width 0.25) (layer "B.Cu") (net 14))
 (segment (start 88.10625 77.60625) (end 89.03125 76.68125) (width 0.25) (layer "B.Cu") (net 14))
 (segment (start 89.03125 73.96525) (end 87.541 72.475) (width 0.25) (layer "B.Cu") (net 14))
 (segment (start 89.03125 76.68125) (end 89.03125 73.96525) (width 0.25) (layer "B.Cu") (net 14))
 (segment (start 91.775 77.60625) (end 88.10625 77.60625) (width 0.25) (layer "B.Cu") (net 14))
 (segment (start 92.075 77.30625) (end 91.775 77.60625) (width 0.25) (layer "B.Cu") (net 14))
 (segment (start 95.25 66.9875) (end 94.1625 65.9) (width 0.25) (layer "B.Cu") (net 20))
 (segment (start 94.1625 65.9) (end 92.441 65.9) (width 0.25) (layer "B.Cu") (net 20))
 (segment (start 76.2 67.46875) (end 75.40625 68.2625) (width 0.25) (layer "F.Cu") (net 10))
 (segment (start 56.35625 68.2625) (end 56.35625 76.2) (width 0.25) (layer "F.Cu") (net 10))
 (segment (start 55.5625 65.0875) (end 55.5625 67.46875) (width 0.25) (layer "F.Cu") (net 10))
 (segment (start 55.5625 67.46875) (end 56.35625 68.2625) (width 0.25) (layer "F.Cu") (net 10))
 (segment (start 75.40625 68.2625) (end 56.35625 68.2625) (width 0.25) (layer "F.Cu") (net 10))
 (via (at 55.5625 65.0875) (size 0.8) (drill 0.4) (layers "F.Cu" "B.Cu") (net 10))
 (via (at 76.2 67.46875) (size 0.8) (drill 0.4) (layers "F.Cu" "B.Cu") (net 10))
 (via (at 56.35625 76.2) (size 0.8) (drill 0.4) (layers "F.Cu" "B.Cu") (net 10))
 (segment (start 81.041 66.7) (end 76.96875 66.7) (width 0.25) (layer "B.Cu") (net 10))
 (segment (start 56.041 76.2) (end 55.626 76.615) (width 0.25) (layer "B.Cu") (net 10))
 (segment (start 55.626 57.565) (end 55.5625 57.6285) (width 0.25) (layer "B.Cu") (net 10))
 (segment (start 76.96875 66.7) (end 76.2 67.46875) (width 0.25) (layer "B.Cu") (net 10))
 (segment (start 55.5625 57.6285) (end 55.5625 65.0875) (width 0.25) (layer "B.Cu") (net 10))
 (segment (start 56.35625 76.2) (end 56.041 76.2) (width 0.25) (layer "B.Cu") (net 10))
 (segment (start 53.467 53.306) (end 55.626 55.465) (width 0.25) (layer "B.Cu") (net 6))
 (segment (start 53.467 51.435) (end 53.467 53.306) (width 0.25) (layer "B.Cu") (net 6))
 (segment (start 74.6125 73.025) (end 74.6125 65.0875) (width 0.25) (layer "B.Cu") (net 9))
 (segment (start 75.226 76.065) (end 75.226 73.6385) (width 0.25) (layer "B.Cu") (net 9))
 (segment (start 74.676 63.5635) (end 75.40625 64.29375) (width 0.25) (layer "B.Cu") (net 9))
 (segment (start 74.676 57.565) (end 74.676 63.5635) (width 0.25) (layer "B.Cu") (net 9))
 (segment (start 75.40625 64.29375) (end 79.375 64.29375) (width 0.25) (layer "B.Cu") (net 9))
 (segment (start 74.6125 65.0875) (end 75.40625 64.29375) (width 0.25) (layer "B.Cu") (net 9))
 (segment (start 75.226 73.6385) (end 74.6125 73.025) (width 0.25) (layer "B.Cu") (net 9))
 (segment (start 79.375 64.29375) (end 79.38125 64.3) (width 0.25) (layer "B.Cu") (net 9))
 (segment (start 74.676 76.615) (end 75.226 76.065) (width 0.25) (layer "B.Cu") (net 9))
 (segment (start 79.38125 64.3) (end 81.041 64.3) (width 0.25) (layer "B.Cu") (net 9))
 (segment (start 72.517 53.306) (end 74.676 55.465) (width 0.25) (layer "B.Cu") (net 5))
 (segment (start 72.517 51.435) (end 72.517 53.306) (width 0.25) (layer "B.Cu") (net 5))
 (segment (start 53.467 72.356) (end 55.626 74.515) (width 0.25) (layer "B.Cu") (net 3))
 (segment (start 53.467 70.485) (end 53.467 72.356) (width 0.25) (layer "B.Cu") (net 3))
 (segment (start 72.517 72.356) (end 74.676 74.515) (width 0.25) (layer "B.Cu") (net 2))
 (segment (start 72.517 70.485) (end 72.517 72.356) (width 0.25) (layer "B.Cu") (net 2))
 (segment (start 94.759342 54.503342) (end 93.15625 52.90025) (width 0.381) (layer "B.Cu") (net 15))
 (segment (start 98.425 56.95625) (end 95.972092 54.503342) (width 0.381) (layer "B.Cu") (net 15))
 (segment (start 95.972092 54.503342) (end 94.759342 54.503342) (width 0.381) (layer "B.Cu") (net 15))
 (segment (start 98.425 65.88125) (end 98.425 56.95625) (width 0.381) (layer "B.Cu") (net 15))
 (segment (start 93.15625 52.90025) (end 93.15625 50.285) (width 0.381) (layer "B.Cu") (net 15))
 (segment (start 95.25 53.975) (end 95.25 55.5625) (width 0.2) (layer "F.Cu") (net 16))
 (segment (start 93.94625 52.3875) (end 93.94625 52.67125) (width 0.2) (layer "F.Cu") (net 16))
 (segment (start 93.94625 52.67125) (end 95.25 53.975) (width 0.2) (layer "F.Cu") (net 16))
 (via (at 93.94625 52.3875) (size 0.8) (drill 0.4) (layers "F.Cu" "B.Cu") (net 16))
 (via (at 95.25 55.5625) (size 0.8) (drill 0.4) (layers "F.Cu" "B.Cu") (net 16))
 (segment (start 93.80625 50.285) (end 93.80625 52.2475) (width 0.2) (layer "B.Cu") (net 16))
 (segment (start 95.25 57.15) (end 95.25625 57.14375) (width 0.2) (layer "B.Cu") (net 16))
 (segment (start 95.25 55.5625) (end 95.25 57.15) (width 0.2) (layer "B.Cu") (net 16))
 (segment (start 93.80625 52.2475) (end 93.94625 52.3875) (width 0.2) (layer "B.Cu") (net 16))
 (segment (start 96.8375 54.25875) (end 94.96625 52.3875) (width 0.2) (layer "F.Cu") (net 11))
 (segment (start 96.8375 59.53125) (end 96.8375 54.25875) (width 0.2) (layer "F.Cu") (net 11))
 (via (at 96.8375 59.53125) (size 0.8) (drill 0.4) (layers "F.Cu" "B.Cu") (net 11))
 (via (at 94.96625 52.3875) (size 0.8) (drill 0.4) (layers "F.Cu" "B.Cu") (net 11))
 (segment (start 94.45625 50.285) (end 94.45625 51.8775) (width 0.2) (layer "B.Cu") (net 11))
 (segment (start 94.45625 51.8775) (end 94.96625 52.3875) (width 0.2) (layer "B.Cu") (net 11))
 (segment (start 96.8375 59.53125) (end 95.25 61.11875) (width 0.2) (layer "B.Cu") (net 11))
 (segment (start 73.025 65.88125) (end 73.81875 65.0875) (width 0.25) (layer "F.Cu") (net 4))
 (segment (start 73.81875 65.0875) (end 76.2 65.0875) (width 0.25) (layer "F.Cu") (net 4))
 (segment (start 55.5625 53.975) (end 47.625 53.975) (width 0.25) (layer "F.Cu") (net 4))
 (segment (start 47.625 53.975) (end 45.24375 51.59375) (width 0.25) (layer "F.Cu") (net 4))
 (via (at 55.5625 53.975) (size 0.8) (drill 0.4) (layers "F.Cu" "B.Cu") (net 4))
 (via (at 45.24375 51.59375) (size 0.8) (drill 0.4) (layers "F.Cu" "B.Cu") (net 4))
 (via (at 73.025 65.88125) (size 0.8) (drill 0.4) (layers "F.Cu" "B.Cu") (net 4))
 (via (at 76.2 65.0875) (size 0.8) (drill 0.4) (layers "F.Cu" "B.Cu") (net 4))
 (segment (start 41.275 65.88125) (end 65.441032 65.88125) (width 0.25) (layer "B.Cu") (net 4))
 (segment (start 42.92125 51.59375) (end 40.54 53.975) (width 0.25) (layer "B.Cu") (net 4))
 (segment (start 40.54 56.277767) (end 40.48125 56.336517) (width 0.25) (layer "B.Cu") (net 4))
 (segment (start 40.54 53.975) (end 40.54 56.277767) (width 0.25) (layer "B.Cu") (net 4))
 (segment (start 76.2125 65.1) (end 81.041 65.1) (width 0.25) (layer "B.Cu") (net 4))
 (segment (start 59.59 53.975) (end 55.5625 53.975) (width 0.25) (layer "B.Cu") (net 4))
 (segment (start 65.441032 65.88125) (end 73.025 65.88125) (width 0.25) (layer "B.Cu") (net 4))
 (segment (start 40.48125 65.0875) (end 41.275 65.88125) (width 0.25) (layer "B.Cu") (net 4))
 (segment (start 45.24375 51.59375) (end 42.92125 51.59375) (width 0.25) (layer "B.Cu") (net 4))
 (segment (start 40.48125 56.336517) (end 40.48125 65.0875) (width 0.25) (layer "B.Cu") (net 4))
 (segment (start 76.2 65.0875) (end 76.2125 65.1) (width 0.25) (layer "B.Cu") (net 4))
 (segment (start 75.200497 66.880753) (end 76.2 65.88125) (width 0.25) (layer "F.Cu") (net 1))
 (segment (start 76.2 66.087003) (end 76.2 65.88125) (width 0.25) (layer "F.Cu") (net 1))
 (segment (start 45.24375 70.64375) (end 47.625 73.025) (width 0.25) (layer "F.Cu") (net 1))
 (segment (start 47.625 73.025) (end 55.5625 73.025) (width 0.25) (layer "F.Cu") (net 1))
 (segment (start 73.025 66.880753) (end 75.200497 66.880753) (width 0.25) (layer "F.Cu") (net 1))
 (via (at 55.5625 73.025) (size 0.8) (drill 0.4) (layers "F.Cu" "B.Cu") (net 1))
 (via (at 45.24375 70.64375) (size 0.8) (drill 0.4) (layers "F.Cu" "B.Cu") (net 1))
 (via (at 73.025 66.880753) (size 0.8) (drill 0.4) (layers "F.Cu" "B.Cu") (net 1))
 (via (at 76.2 66.087003) (size 0.8) (drill 0.4) (layers "F.Cu" "B.Cu") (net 1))
 (segment (start 40.54 73.025) (end 42.92125 70.64375) (width 0.25) (layer "B.Cu") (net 1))
 (segment (start 41.275 66.675) (end 73.025 66.675) (width 0.25) (layer "B.Cu") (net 1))
 (segment (start 40.54 73.025) (end 40.54 67.41) (width 0.25) (layer "B.Cu") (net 1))
 (segment (start 40.54 67.41) (end 41.275 66.675) (width 0.25) (layer "B.Cu") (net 1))
 (segment (start 73.025 66.675) (end 73.025 66.880753) (width 0.25) (layer "B.Cu") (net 1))
 (segment (start 42.92125 70.64375) (end 45.24375 70.64375) (width 0.25) (layer "B.Cu") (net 1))
 (segment (start 76.2 66.087003) (end 76.387003 65.9) (width 0.25) (layer "B.Cu") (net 1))
 (segment (start 76.387003 65.9) (end 81.041 65.9) (width 0.25) (layer "B.Cu") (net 1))
 (segment (start 55.5625 73.025) (end 59.59 73.025) (width 0.25) (layer "B.Cu") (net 1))
 (segment (start 93.825 63.116) (end 93.825 59.94271) (width 0.25) (layer "B.Cu") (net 23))
 (segment (start 92.441 63.5) (end 93.441 63.5) (width 0.25) (layer "B.Cu") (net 23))
 (segment (start 94.79271 58.975) (end 95.25 58.975) (width 0.25) (layer "B.Cu") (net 23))
 (segment (start 93.825 59.94271) (end 94.79271 58.975) (width 0.25) (layer "B.Cu") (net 23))
 (segment (start 93.441 63.5) (end 93.825 63.116) (width 0.25) (layer "B.Cu") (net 23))
 (segment (start 93.89375 64.3) (end 92.441 64.3) (width 0.25) (layer "B.Cu") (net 12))
 (segment (start 95.25 62.94375) (end 93.89375 64.3) (width 0.25) (layer "B.Cu") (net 12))
 (segment (start 95.175 70.95625) (end 95.25 70.88125) (width 0.25) (layer "B.Cu") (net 19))
 (segment (start 90.491 73.025) (end 89.941 72.475) (width 0.25) (layer "B.Cu") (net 19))
 (segment (start 95.175 79.90625) (end 95.175 73.025) (width 0.25) (layer "B.Cu") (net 19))
 (segment (start 95.175 73.025) (end 95.175 70.95625) (width 0.25) (layer "B.Cu") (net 19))
 (segment (start 89.941 72.475) (end 89.941 71.6) (width 0.25) (layer "B.Cu") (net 19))
 (segment (start 95.175 73.025) (end 90.491 73.025) (width 0.25) (layer "B.Cu") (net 19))
 (segment (start 77.8 61.9) (end 81.041 61.9) (width 0.25) (layer "B.Cu") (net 21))
 (segment (start 77.7875 61.9125) (end 77.8 61.9) (width 0.25) (layer "B.Cu") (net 21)))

